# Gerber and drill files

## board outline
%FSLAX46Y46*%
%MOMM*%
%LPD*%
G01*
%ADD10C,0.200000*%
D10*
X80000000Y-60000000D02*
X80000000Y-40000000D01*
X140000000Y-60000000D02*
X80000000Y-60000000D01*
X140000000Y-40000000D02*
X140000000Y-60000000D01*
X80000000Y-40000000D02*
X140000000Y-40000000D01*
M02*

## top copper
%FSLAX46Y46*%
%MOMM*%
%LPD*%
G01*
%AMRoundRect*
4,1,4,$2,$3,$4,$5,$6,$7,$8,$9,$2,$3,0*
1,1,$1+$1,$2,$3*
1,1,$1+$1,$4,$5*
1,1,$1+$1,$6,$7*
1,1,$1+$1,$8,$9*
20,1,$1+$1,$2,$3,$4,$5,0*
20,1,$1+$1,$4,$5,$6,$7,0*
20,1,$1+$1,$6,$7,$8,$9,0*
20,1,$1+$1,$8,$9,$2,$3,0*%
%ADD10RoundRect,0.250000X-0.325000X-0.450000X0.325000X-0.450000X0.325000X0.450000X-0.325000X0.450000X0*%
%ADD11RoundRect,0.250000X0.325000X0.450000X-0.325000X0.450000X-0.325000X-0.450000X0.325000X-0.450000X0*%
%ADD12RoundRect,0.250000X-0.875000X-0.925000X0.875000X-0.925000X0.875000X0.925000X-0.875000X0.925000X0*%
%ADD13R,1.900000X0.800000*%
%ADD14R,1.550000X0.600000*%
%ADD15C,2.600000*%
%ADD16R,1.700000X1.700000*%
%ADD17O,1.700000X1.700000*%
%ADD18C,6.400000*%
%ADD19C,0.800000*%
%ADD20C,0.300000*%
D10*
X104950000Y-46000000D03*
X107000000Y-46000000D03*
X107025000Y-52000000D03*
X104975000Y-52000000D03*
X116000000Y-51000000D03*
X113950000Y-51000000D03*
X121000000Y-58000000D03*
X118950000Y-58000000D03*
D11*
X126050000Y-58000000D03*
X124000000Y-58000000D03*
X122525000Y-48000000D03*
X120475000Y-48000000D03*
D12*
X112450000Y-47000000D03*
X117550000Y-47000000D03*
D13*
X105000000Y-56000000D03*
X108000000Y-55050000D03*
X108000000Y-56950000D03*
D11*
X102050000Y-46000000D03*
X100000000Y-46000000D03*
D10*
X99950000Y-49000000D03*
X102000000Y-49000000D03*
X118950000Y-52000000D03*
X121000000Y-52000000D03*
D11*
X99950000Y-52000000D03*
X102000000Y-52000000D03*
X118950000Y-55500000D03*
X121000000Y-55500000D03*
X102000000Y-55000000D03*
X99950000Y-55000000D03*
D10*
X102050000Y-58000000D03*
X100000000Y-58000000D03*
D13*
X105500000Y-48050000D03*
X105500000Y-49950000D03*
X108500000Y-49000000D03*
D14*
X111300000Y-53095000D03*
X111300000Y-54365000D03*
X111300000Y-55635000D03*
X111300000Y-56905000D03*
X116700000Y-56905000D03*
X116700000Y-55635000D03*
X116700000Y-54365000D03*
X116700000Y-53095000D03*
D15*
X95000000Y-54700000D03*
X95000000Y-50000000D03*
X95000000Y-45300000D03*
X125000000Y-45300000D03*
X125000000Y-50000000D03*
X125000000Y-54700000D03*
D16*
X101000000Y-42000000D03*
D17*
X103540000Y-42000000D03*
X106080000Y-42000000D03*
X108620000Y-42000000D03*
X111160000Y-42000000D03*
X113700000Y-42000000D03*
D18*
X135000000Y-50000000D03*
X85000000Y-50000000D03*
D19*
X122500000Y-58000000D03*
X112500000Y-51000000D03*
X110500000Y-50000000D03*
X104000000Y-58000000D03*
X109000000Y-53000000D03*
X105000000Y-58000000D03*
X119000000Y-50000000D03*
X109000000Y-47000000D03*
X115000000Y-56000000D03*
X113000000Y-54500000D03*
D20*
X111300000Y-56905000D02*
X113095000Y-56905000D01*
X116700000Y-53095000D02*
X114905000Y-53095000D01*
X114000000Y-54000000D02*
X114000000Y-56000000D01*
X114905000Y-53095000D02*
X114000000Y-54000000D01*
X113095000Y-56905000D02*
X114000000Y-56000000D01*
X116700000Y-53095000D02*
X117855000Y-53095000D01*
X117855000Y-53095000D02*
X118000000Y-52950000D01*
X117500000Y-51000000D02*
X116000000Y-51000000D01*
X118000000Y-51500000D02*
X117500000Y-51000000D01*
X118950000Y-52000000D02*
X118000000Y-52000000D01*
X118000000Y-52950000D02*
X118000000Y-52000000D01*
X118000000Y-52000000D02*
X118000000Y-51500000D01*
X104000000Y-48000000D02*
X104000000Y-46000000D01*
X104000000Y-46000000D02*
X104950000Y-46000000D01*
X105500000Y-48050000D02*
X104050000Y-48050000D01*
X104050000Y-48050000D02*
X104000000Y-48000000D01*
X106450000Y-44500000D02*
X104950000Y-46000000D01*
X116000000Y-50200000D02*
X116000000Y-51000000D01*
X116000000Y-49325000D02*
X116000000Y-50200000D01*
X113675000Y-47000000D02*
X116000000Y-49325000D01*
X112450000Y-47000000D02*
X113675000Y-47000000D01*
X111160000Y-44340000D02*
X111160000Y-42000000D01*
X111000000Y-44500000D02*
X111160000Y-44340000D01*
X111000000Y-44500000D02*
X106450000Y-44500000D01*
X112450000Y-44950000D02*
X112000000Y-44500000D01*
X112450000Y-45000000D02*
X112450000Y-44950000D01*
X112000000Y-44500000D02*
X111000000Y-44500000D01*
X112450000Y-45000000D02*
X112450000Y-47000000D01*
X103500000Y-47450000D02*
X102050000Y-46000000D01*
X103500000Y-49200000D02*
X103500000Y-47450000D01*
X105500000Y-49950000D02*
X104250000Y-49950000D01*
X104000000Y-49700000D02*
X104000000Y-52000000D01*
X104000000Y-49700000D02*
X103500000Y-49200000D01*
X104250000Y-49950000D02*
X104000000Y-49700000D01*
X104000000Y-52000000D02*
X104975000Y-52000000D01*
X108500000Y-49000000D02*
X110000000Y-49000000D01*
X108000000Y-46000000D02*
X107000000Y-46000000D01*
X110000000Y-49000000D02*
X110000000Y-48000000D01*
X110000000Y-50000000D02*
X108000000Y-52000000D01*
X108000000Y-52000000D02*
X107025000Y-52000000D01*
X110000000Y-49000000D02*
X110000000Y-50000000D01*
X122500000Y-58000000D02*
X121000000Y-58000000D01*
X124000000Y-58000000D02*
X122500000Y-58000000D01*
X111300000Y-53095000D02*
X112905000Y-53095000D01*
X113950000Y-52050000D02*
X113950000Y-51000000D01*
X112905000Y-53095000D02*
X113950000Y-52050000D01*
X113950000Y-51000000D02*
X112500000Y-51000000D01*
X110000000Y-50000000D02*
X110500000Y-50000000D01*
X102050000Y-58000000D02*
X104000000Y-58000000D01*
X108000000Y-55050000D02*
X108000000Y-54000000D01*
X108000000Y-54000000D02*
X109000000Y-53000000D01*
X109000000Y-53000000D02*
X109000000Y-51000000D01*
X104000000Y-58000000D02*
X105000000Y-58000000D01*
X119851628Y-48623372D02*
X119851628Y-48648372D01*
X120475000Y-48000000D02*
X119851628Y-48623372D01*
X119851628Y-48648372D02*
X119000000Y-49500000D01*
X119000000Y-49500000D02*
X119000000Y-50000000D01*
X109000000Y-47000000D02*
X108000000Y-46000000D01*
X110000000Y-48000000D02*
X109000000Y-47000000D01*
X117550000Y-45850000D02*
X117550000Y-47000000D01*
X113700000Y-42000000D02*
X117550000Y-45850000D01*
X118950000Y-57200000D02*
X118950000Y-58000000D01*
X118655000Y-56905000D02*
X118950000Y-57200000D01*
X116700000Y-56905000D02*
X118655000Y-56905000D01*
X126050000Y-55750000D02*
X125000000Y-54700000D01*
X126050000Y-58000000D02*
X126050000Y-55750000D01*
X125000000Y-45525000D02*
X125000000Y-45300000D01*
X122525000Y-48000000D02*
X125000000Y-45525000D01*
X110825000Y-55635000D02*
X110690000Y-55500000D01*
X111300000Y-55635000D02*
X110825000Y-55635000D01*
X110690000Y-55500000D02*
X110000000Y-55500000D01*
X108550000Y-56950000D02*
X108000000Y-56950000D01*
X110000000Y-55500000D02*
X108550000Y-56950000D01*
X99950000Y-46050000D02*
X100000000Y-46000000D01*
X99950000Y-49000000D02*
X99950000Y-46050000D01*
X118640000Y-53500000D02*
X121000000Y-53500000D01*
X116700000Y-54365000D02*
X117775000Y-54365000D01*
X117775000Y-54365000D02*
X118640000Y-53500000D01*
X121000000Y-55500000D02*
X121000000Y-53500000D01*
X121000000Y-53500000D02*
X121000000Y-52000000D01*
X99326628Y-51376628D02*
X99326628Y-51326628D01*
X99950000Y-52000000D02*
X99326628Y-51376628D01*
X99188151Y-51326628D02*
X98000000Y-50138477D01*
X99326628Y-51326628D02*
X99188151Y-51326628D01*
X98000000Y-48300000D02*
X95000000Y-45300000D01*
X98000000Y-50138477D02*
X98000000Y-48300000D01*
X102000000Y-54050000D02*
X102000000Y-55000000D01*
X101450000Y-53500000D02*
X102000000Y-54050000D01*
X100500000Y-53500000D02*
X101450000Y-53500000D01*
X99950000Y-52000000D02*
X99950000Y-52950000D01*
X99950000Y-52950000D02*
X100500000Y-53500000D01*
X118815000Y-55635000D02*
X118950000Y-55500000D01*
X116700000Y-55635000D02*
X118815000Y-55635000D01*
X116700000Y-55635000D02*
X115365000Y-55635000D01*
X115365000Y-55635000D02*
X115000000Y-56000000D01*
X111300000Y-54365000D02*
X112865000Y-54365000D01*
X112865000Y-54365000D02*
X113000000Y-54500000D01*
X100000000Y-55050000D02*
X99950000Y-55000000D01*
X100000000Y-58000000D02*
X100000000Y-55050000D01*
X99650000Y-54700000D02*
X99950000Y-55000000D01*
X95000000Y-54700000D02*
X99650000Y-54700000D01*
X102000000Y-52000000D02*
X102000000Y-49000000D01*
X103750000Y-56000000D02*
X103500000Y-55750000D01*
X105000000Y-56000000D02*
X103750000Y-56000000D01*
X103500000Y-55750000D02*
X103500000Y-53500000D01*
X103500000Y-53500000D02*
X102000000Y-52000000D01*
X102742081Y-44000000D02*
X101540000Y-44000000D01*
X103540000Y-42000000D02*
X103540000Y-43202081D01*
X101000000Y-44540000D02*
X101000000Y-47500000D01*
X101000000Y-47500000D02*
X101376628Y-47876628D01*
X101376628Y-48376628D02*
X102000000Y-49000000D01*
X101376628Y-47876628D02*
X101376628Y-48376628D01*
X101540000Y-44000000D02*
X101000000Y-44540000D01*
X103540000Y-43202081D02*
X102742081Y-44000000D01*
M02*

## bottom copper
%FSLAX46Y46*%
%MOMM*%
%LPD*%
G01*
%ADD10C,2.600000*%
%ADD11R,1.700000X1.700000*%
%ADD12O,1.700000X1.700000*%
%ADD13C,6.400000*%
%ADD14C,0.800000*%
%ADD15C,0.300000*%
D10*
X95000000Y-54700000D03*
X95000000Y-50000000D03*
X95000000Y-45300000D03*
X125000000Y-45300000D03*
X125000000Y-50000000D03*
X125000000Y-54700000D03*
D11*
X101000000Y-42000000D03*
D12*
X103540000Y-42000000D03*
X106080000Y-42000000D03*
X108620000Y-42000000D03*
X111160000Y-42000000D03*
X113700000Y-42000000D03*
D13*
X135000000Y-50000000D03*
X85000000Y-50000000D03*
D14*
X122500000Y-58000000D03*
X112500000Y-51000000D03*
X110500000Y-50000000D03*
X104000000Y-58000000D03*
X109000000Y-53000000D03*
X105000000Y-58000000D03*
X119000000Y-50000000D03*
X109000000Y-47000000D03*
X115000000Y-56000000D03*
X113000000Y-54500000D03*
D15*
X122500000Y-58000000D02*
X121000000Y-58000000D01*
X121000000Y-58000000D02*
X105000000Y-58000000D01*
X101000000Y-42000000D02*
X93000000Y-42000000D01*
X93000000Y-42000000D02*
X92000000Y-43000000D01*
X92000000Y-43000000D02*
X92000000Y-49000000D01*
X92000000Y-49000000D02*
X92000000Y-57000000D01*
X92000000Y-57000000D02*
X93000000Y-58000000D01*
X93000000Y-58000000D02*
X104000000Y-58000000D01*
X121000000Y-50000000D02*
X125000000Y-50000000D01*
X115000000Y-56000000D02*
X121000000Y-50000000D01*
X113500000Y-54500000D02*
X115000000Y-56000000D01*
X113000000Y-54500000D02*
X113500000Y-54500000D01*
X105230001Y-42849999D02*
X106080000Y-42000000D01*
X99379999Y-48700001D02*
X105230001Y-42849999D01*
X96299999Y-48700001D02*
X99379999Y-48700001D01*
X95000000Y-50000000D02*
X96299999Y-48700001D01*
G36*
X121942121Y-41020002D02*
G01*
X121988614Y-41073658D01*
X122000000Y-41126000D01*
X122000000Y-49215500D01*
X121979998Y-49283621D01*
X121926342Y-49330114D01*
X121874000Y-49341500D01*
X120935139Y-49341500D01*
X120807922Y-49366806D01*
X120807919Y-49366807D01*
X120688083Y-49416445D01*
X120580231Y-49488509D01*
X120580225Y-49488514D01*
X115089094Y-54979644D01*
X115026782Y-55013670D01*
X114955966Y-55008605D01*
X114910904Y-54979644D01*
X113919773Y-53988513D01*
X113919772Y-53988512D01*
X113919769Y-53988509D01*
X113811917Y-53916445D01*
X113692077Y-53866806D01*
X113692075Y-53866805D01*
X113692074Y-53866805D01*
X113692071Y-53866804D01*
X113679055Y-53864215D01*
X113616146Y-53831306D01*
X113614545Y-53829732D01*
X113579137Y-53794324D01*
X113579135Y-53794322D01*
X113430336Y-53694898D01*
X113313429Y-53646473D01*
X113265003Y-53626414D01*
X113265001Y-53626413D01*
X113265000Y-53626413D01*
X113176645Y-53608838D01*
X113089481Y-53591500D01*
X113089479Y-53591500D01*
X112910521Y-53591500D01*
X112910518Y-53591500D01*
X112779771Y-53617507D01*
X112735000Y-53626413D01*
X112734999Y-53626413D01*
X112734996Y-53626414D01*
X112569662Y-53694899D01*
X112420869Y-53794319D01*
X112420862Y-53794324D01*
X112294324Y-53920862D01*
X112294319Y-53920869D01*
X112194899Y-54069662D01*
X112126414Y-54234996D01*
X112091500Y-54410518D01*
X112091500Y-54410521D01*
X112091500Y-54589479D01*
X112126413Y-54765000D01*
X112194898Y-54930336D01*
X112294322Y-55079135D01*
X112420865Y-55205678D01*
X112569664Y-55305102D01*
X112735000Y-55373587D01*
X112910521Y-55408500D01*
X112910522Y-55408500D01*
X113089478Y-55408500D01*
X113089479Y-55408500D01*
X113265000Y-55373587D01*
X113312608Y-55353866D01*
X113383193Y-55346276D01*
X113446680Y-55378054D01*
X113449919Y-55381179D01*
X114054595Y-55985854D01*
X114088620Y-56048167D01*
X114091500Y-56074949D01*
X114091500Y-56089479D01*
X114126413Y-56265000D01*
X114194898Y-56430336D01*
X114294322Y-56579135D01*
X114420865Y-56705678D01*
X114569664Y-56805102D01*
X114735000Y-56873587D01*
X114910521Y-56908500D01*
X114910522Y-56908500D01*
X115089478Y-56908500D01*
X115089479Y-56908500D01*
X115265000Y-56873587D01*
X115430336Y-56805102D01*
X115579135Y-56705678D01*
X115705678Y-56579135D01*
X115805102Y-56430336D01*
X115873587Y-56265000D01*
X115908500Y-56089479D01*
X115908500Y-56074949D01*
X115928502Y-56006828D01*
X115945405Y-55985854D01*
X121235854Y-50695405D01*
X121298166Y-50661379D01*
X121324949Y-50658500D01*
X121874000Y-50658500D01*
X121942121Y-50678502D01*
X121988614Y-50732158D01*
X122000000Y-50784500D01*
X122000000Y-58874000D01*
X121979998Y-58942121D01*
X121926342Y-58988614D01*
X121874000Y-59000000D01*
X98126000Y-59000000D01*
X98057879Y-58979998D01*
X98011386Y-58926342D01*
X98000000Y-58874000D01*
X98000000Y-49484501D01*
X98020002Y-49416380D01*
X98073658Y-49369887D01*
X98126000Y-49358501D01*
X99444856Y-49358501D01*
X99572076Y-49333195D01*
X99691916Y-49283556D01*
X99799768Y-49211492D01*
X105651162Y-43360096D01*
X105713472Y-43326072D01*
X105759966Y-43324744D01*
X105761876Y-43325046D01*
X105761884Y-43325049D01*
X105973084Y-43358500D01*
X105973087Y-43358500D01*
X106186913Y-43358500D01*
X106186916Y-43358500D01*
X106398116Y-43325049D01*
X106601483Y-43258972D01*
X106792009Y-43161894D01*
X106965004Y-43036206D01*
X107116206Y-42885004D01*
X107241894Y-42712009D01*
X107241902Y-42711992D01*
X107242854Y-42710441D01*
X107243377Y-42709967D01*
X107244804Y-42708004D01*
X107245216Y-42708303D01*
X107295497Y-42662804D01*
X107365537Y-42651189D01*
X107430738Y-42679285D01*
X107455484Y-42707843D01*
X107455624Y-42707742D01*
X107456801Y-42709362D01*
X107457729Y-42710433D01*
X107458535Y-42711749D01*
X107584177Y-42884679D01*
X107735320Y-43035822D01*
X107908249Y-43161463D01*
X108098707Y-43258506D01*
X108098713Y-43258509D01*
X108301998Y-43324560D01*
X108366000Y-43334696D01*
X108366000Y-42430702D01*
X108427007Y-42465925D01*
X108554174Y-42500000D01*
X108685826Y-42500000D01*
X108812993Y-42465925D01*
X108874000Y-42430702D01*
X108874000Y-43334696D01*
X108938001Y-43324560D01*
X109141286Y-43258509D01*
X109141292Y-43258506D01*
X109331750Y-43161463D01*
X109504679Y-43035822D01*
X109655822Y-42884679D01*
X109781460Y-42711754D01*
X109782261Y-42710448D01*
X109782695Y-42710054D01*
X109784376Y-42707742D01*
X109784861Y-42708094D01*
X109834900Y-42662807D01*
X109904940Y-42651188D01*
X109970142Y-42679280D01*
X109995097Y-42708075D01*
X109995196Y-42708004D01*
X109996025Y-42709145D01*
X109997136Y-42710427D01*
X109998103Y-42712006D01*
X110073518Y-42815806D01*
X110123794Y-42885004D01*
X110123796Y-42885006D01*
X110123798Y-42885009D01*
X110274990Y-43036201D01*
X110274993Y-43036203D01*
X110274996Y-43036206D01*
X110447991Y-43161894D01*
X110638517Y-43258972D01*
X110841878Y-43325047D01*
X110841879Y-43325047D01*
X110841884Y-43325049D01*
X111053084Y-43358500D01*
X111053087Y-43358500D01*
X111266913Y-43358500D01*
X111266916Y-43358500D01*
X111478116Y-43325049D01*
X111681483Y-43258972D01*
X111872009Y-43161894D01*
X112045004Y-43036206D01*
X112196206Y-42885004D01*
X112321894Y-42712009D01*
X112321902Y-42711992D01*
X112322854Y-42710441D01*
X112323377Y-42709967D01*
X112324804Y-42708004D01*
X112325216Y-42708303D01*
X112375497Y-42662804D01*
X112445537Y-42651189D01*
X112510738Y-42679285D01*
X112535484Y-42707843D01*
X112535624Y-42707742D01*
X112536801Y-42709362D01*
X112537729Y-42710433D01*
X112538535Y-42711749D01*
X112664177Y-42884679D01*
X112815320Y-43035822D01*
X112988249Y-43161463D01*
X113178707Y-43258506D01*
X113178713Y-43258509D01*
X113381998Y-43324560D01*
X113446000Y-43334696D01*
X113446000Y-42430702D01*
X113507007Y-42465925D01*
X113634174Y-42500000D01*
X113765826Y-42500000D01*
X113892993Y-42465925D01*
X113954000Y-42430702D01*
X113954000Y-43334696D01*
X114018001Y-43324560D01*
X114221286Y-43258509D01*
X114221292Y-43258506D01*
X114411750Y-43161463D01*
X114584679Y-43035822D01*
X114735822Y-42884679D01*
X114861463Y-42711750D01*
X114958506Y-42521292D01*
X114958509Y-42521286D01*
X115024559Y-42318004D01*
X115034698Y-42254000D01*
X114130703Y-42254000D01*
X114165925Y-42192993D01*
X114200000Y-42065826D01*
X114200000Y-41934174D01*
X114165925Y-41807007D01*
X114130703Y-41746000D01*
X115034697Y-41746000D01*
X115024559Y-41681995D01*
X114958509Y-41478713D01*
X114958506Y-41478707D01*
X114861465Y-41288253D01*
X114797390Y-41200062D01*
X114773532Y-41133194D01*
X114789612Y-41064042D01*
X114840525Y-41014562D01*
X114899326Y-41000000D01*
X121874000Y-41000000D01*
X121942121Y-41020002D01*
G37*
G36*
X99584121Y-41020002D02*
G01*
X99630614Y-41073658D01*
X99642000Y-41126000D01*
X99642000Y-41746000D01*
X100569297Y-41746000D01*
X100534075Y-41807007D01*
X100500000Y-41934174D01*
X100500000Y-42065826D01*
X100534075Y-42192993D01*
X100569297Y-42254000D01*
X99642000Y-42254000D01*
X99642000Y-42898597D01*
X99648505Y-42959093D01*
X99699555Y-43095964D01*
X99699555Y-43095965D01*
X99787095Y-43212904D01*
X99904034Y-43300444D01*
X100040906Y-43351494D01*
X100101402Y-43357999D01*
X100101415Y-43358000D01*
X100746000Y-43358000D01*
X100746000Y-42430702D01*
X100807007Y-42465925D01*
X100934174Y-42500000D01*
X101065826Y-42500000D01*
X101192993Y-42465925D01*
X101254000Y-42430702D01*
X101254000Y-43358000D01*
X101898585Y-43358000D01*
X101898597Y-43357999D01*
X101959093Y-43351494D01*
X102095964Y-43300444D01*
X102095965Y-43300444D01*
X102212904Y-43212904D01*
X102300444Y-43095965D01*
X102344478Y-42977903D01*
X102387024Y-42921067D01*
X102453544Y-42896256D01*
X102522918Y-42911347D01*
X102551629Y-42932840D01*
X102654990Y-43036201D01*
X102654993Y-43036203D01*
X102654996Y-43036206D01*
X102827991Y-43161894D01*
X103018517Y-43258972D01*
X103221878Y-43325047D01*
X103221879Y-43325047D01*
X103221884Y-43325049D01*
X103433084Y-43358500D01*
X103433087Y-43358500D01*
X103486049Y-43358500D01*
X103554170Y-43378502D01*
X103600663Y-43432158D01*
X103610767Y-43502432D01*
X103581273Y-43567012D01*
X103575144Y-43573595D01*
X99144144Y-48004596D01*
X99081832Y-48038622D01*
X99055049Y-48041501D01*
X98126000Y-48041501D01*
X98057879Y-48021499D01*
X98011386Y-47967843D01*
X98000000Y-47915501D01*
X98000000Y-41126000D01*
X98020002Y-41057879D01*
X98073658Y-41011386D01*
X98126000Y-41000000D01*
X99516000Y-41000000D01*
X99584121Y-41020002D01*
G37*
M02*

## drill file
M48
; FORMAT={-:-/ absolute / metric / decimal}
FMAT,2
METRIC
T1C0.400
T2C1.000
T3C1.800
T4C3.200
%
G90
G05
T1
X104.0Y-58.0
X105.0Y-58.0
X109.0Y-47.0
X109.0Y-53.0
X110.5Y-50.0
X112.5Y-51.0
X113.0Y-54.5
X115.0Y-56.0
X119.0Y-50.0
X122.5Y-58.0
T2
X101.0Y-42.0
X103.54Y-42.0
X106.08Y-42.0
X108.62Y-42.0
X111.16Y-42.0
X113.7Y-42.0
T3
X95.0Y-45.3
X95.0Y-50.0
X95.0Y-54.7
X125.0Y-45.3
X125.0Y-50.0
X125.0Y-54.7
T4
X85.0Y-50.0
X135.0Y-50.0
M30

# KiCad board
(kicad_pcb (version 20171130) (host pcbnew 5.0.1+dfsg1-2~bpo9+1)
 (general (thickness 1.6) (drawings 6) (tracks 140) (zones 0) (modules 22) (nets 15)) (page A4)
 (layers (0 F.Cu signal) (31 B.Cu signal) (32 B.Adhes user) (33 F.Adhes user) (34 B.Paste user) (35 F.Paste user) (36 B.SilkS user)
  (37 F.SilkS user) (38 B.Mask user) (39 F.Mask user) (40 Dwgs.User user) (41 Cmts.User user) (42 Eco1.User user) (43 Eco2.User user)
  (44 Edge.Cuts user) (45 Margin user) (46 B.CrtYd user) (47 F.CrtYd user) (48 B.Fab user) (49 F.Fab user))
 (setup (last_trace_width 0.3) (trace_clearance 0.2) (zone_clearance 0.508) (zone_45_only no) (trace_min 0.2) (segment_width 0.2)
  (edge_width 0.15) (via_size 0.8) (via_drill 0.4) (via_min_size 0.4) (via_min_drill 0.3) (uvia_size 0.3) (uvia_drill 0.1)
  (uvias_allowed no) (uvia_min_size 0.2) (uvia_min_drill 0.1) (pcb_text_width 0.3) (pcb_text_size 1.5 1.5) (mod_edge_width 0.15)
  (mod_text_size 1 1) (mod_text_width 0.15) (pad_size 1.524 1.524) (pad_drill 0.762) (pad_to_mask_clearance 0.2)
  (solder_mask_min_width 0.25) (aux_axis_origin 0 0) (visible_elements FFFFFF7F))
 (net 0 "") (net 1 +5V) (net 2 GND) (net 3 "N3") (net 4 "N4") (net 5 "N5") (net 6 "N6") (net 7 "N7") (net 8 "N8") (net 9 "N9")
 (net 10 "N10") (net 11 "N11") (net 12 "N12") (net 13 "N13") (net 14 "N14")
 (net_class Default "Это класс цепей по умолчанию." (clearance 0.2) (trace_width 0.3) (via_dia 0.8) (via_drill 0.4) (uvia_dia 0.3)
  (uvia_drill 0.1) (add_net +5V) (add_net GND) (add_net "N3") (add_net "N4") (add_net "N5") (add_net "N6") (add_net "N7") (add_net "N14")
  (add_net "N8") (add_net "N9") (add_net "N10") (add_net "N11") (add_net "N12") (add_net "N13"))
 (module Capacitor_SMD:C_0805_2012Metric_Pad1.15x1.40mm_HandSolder (layer F.Cu) (at 105.975 46)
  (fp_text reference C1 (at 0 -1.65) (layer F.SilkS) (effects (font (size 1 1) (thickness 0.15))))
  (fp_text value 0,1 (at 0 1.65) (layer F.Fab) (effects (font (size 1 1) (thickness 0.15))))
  (pad 1 smd roundrect (at -1.025 0) (size 1.15 1.4) (layers F.Cu F.Paste F.Mask) (roundrect_rratio 0.217391) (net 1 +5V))
  (pad 2 smd roundrect (at 1.025 0) (size 1.15 1.4) (layers F.Cu F.Paste F.Mask) (roundrect_rratio 0.217391) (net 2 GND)))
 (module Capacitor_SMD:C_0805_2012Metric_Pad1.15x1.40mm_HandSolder (layer F.Cu) (at 106 52)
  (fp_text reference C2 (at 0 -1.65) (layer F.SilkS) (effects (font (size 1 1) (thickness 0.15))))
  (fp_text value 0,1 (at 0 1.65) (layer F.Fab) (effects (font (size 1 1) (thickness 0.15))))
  (pad 2 smd roundrect (at 1.025 0) (size 1.15 1.4) (layers F.Cu F.Paste F.Mask) (roundrect_rratio 0.217391) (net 2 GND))
  (pad 1 smd roundrect (at -1.025 0) (size 1.15 1.4) (layers F.Cu F.Paste F.Mask) (roundrect_rratio 0.217391) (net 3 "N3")))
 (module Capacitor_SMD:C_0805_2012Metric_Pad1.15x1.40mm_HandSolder (layer F.Cu) (at 114.975 51)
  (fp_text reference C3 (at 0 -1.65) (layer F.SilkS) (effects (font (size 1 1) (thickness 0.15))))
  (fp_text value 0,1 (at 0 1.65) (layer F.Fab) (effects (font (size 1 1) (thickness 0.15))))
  (pad 2 smd roundrect (at 1.025 0) (size 1.15 1.4) (layers F.Cu F.Paste F.Mask) (roundrect_rratio 0.217391) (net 1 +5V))
  (pad 1 smd roundrect (at -1.025 0) (size 1.15 1.4) (layers F.Cu F.Paste F.Mask) (roundrect_rratio 0.217391) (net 2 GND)))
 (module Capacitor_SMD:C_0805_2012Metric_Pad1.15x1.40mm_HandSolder (layer F.Cu) (at 119.975 58)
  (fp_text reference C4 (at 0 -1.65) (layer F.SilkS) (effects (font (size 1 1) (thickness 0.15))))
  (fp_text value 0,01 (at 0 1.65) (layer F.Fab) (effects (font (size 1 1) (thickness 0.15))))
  (pad 2 smd roundrect (at 1.025 0) (size 1.15 1.4) (layers F.Cu F.Paste F.Mask) (roundrect_rratio 0.217391) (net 2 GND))
  (pad 1 smd roundrect (at -1.025 0) (size 1.15 1.4) (layers F.Cu F.Paste F.Mask) (roundrect_rratio 0.217391) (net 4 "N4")))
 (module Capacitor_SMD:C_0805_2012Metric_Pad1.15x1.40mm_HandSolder (layer F.Cu) (at 125.025 58 180)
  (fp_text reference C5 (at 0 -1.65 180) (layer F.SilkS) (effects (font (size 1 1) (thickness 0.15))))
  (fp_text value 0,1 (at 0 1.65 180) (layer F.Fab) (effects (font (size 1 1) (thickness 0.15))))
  (pad 1 smd roundrect (at -1.025 0 180) (size 1.15 1.4) (layers F.Cu F.Paste F.Mask) (roundrect_rratio 0.217391) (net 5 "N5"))
  (pad 2 smd roundrect (at 1.025 0 180) (size 1.15 1.4) (layers F.Cu F.Paste F.Mask) (roundrect_rratio 0.217391) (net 2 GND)))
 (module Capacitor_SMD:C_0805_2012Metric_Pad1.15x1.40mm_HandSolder (layer F.Cu) (at 121.5 48 180)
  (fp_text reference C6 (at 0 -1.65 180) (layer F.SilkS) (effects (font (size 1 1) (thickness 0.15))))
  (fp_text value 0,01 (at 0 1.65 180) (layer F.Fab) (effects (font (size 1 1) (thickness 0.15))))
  (pad 1 smd roundrect (at -1.025 0 180) (size 1.15 1.4) (layers F.Cu F.Paste F.Mask) (roundrect_rratio 0.217391) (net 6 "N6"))
  (pad 2 smd roundrect (at 1.025 0 180) (size 1.15 1.4) (layers F.Cu F.Paste F.Mask) (roundrect_rratio 0.217391) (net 2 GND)))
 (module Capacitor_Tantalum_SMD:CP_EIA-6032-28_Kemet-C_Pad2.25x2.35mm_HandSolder (layer F.Cu) (at 115 47)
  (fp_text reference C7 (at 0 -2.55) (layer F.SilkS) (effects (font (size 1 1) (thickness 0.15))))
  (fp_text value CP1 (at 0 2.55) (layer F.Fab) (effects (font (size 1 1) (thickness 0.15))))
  (pad 1 smd roundrect (at -2.55 0) (size 2.25 2.35) (layers F.Cu F.Paste F.Mask) (roundrect_rratio 0.111111) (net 1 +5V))
  (pad 2 smd roundrect (at 2.55 0) (size 2.25 2.35) (layers F.Cu F.Paste F.Mask) (roundrect_rratio 0.111111) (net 2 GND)))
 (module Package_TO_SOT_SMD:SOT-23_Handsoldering (layer F.Cu) (at 106.5 56 180)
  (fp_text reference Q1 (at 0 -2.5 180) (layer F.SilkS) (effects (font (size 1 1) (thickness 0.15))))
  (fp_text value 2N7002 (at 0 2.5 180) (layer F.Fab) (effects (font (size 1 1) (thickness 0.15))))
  (pad 3 smd rect (at 1.5 0 180) (size 1.9 0.8) (layers F.Cu F.Paste F.Mask) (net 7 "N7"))
  (pad 2 smd rect (at -1.5 0.95 180) (size 1.9 0.8) (layers F.Cu F.Paste F.Mask) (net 2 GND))
  (pad 1 smd rect (at -1.5 -0.95 180) (size 1.9 0.8) (layers F.Cu F.Paste F.Mask) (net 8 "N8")))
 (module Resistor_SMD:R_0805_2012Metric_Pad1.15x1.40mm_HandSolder (layer F.Cu) (at 101.025 46 180)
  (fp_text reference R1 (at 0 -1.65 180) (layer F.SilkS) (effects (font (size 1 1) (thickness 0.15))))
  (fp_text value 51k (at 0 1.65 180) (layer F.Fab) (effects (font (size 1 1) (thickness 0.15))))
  (pad 1 smd roundrect (at -1.025 0 180) (size 1.15 1.4) (layers F.Cu F.Paste F.Mask) (roundrect_rratio 0.217391) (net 3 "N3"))
  (pad 2 smd roundrect (at 1.025 0 180) (size 1.15 1.4) (layers F.Cu F.Paste F.Mask) (roundrect_rratio 0.217391) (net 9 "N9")))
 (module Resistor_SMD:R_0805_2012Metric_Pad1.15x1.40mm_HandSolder (layer F.Cu) (at 100.975 49)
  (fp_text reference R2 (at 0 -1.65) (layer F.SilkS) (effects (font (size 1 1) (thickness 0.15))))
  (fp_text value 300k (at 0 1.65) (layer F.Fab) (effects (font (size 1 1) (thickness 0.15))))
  (pad 1 smd roundrect (at -1.025 0) (size 1.15 1.4) (layers F.Cu F.Paste F.Mask) (roundrect_rratio 0.217391) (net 9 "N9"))
  (pad 2 smd roundrect (at 1.025 0) (size 1.15 1.4) (layers F.Cu F.Paste F.Mask) (roundrect_rratio 0.217391) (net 7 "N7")))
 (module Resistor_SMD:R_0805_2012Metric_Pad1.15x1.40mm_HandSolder (layer F.Cu) (at 119.975 52)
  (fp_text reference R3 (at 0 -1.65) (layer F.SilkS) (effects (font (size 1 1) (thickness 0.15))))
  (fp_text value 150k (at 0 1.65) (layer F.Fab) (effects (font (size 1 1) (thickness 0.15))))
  (pad 1 smd roundrect (at -1.025 0) (size 1.15 1.4) (layers F.Cu F.Paste F.Mask) (roundrect_rratio 0.217391) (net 1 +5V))
  (pad 2 smd roundrect (at 1.025 0) (size 1.15 1.4) (layers F.Cu F.Paste F.Mask) (roundrect_rratio 0.217391) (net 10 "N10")))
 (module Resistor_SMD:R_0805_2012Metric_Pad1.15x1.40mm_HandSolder (layer F.Cu) (at 100.975 52 180)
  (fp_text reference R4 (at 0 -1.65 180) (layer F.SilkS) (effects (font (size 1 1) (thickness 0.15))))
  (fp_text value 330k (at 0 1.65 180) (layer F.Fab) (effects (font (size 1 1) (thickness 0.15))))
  (pad 2 smd roundrect (at 1.025 0 180) (size 1.15 1.4) (layers F.Cu F.Paste F.Mask) (roundrect_rratio 0.217391) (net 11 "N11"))
  (pad 1 smd roundrect (at -1.025 0 180) (size 1.15 1.4) (layers F.Cu F.Paste F.Mask) (roundrect_rratio 0.217391) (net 7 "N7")))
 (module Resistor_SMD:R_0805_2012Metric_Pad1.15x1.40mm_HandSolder (layer F.Cu) (at 119.975 55.5 180)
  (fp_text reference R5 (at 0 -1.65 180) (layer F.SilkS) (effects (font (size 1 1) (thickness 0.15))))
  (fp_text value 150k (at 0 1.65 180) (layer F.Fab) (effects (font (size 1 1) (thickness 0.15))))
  (pad 2 smd roundrect (at 1.025 0 180) (size 1.15 1.4) (layers F.Cu F.Paste F.Mask) (roundrect_rratio 0.217391) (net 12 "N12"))
  (pad 1 smd roundrect (at -1.025 0 180) (size 1.15 1.4) (layers F.Cu F.Paste F.Mask) (roundrect_rratio 0.217391) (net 10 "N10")))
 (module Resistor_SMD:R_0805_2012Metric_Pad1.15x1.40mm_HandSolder (layer F.Cu) (at 100.975 55 180)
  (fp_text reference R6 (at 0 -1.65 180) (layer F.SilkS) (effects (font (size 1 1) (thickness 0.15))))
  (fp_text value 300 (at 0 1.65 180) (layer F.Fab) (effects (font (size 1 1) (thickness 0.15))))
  (pad 1 smd roundrect (at -1.025 0 180) (size 1.15 1.4) (layers F.Cu F.Paste F.Mask) (roundrect_rratio 0.217391) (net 11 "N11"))
  (pad 2 smd roundrect (at 1.025 0 180) (size 1.15 1.4) (layers F.Cu F.Paste F.Mask) (roundrect_rratio 0.217391) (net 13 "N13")))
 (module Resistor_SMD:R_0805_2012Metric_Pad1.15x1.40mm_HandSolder (layer F.Cu) (at 101.025 58)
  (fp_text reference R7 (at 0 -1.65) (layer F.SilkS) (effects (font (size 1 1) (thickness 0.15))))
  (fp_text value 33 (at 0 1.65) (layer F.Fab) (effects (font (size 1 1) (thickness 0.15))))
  (pad 2 smd roundrect (at 1.025 0) (size 1.15 1.4) (layers F.Cu F.Paste F.Mask) (roundrect_rratio 0.217391) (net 2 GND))
  (pad 1 smd roundrect (at -1.025 0) (size 1.15 1.4) (layers F.Cu F.Paste F.Mask) (roundrect_rratio 0.217391) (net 13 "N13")))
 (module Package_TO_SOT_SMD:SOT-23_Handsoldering (layer F.Cu) (at 107 49)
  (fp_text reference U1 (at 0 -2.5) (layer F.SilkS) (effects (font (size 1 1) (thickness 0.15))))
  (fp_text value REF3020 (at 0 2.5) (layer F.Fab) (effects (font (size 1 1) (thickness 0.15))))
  (pad 1 smd rect (at -1.5 -0.95) (size 1.9 0.8) (layers F.Cu F.Paste F.Mask) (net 1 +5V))
  (pad 2 smd rect (at -1.5 0.95) (size 1.9 0.8) (layers F.Cu F.Paste F.Mask) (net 3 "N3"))
  (pad 3 smd rect (at 1.5 0) (size 1.9 0.8) (layers F.Cu F.Paste F.Mask) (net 2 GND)))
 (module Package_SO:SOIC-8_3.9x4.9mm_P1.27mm (layer F.Cu) (at 114 55)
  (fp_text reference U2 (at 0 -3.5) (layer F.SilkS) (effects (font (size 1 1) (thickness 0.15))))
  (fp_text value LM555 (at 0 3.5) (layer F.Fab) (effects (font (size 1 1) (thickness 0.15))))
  (pad 1 smd rect (at -2.7 -1.905) (size 1.55 0.6) (layers F.Cu F.Paste F.Mask) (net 2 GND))
  (pad 2 smd rect (at -2.7 -0.635) (size 1.55 0.6) (layers F.Cu F.Paste F.Mask) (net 12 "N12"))
  (pad 3 smd rect (at -2.7 0.635) (size 1.55 0.6) (layers F.Cu F.Paste F.Mask) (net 8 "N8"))
  (pad 4 smd rect (at -2.7 1.905) (size 1.55 0.6) (layers F.Cu F.Paste F.Mask) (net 1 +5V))
  (pad 5 smd rect (at 2.7 1.905) (size 1.55 0.6) (layers F.Cu F.Paste F.Mask) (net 4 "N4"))
  (pad 6 smd rect (at 2.7 0.635) (size 1.55 0.6) (layers F.Cu F.Paste F.Mask) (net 12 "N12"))
  (pad 7 smd rect (at 2.7 -0.635) (size 1.55 0.6) (layers F.Cu F.Paste F.Mask) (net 10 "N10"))
  (pad 8 smd rect (at 2.7 -1.905) (size 1.55 0.6) (layers F.Cu F.Paste F.Mask) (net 1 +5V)))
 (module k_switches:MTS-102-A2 (layer B.Cu) (at 95 50 270)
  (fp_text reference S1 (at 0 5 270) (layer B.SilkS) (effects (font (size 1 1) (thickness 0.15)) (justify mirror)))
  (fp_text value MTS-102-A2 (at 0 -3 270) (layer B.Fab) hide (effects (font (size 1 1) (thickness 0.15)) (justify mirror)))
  (pad 3 thru_hole circle (at 4.7 0 270) (size 2.6 2.6) (drill 1.8) (layers *.Cu *.Mask) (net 13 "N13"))
  (pad 2 thru_hole circle (at 0 0 270) (size 2.6 2.6) (drill 1.8) (layers *.Cu *.Mask) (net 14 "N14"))
  (pad 1 thru_hole circle (at -4.7 0 270) (size 2.6 2.6) (drill 1.8) (layers *.Cu *.Mask) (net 11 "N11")))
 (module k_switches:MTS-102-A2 (layer B.Cu) (at 125 50 270)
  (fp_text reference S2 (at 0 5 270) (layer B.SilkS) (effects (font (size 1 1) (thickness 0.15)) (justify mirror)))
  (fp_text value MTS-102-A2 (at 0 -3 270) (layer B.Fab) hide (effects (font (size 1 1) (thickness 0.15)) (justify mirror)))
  (pad 1 thru_hole circle (at -4.7 0 270) (size 2.6 2.6) (drill 1.8) (layers *.Cu *.Mask) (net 6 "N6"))
  (pad 2 thru_hole circle (at 0 0 270) (size 2.6 2.6) (drill 1.8) (layers *.Cu *.Mask) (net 12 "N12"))
  (pad 3 thru_hole circle (at 4.7 0 270) (size 2.6 2.6) (drill 1.8) (layers *.Cu *.Mask) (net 5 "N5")))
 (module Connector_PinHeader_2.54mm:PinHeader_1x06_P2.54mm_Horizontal (layer F.Cu) (at 101 42 90)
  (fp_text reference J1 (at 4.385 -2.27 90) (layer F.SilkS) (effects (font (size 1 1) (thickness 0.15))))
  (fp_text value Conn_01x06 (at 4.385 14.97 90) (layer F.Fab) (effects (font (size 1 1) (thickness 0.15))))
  (pad 1 thru_hole rect (at 0 0 90) (size 1.7 1.7) (drill 1) (layers *.Cu *.Mask) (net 2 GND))
  (pad 2 thru_hole oval (at 0 2.54 90) (size 1.7 1.7) (drill 1) (layers *.Cu *.Mask) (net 7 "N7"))
  (pad 3 thru_hole oval (at 0 5.08 90) (size 1.7 1.7) (drill 1) (layers *.Cu *.Mask) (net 14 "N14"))
  (pad 4 thru_hole oval (at 0 7.62 90) (size 1.7 1.7) (drill 1) (layers *.Cu *.Mask) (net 2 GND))
  (pad 5 thru_hole oval (at 0 10.16 90) (size 1.7 1.7) (drill 1) (layers *.Cu *.Mask) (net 1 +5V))
  (pad 6 thru_hole oval (at 0 12.7 90) (size 1.7 1.7) (drill 1) (layers *.Cu *.Mask) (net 2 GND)))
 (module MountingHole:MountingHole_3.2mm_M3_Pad (layer F.Cu) (at 135 50)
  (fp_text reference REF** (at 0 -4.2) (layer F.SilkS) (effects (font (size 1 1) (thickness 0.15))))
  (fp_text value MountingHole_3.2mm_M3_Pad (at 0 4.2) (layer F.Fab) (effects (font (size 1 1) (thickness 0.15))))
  (pad 1 thru_hole circle (at 0 0) (size 6.4 6.4) (drill 3.2) (layers *.Cu *.Mask)))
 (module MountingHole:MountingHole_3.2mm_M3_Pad (layer F.Cu) (at 85 50)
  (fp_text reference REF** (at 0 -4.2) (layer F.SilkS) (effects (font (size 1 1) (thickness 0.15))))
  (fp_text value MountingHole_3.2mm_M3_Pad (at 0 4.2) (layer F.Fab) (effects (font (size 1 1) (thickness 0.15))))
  (pad 1 thru_hole circle (at 0 0) (size 6.4 6.4) (drill 3.2) (layers *.Cu *.Mask)))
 (gr_line (start 80 60) (end 80 40) (layer Edge.Cuts) (width 0.2))
 (gr_line (start 140 60) (end 80 60) (layer Edge.Cuts) (width 0.2))
 (gr_line (start 140 40) (end 140 60) (layer Edge.Cuts) (width 0.2))
 (gr_line (start 80 40) (end 140 40) (layer Edge.Cuts) (width 0.2))
 (segment (start 111.3 56.905) (end 113.095 56.905) (width 0.3) (layer F.Cu) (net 1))
 (segment (start 116.7 53.095) (end 114.905 53.095) (width 0.3) (layer F.Cu) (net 1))
 (segment (start 114 54) (end 114 56) (width 0.3) (layer F.Cu) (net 1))
 (segment (start 114.905 53.095) (end 114 54) (width 0.3) (layer F.Cu) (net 1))
 (segment (start 113.095 56.905) (end 114 56) (width 0.3) (layer F.Cu) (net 1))
 (segment (start 116.7 53.095) (end 117.855 53.095) (width 0.3) (layer F.Cu) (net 1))
 (segment (start 117.855 53.095) (end 118 52.95) (width 0.3) (layer F.Cu) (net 1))
 (segment (start 117.5 51) (end 116 51) (width 0.3) (layer F.Cu) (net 1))
 (segment (start 118 51.5) (end 117.5 51) (width 0.3) (layer F.Cu) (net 1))
 (segment (start 118.95 52) (end 118 52) (width 0.3) (layer F.Cu) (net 1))
 (segment (start 118 52.95) (end 118 52) (width 0.3) (layer F.Cu) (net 1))
 (segment (start 118 52) (end 118 51.5) (width 0.3) (layer F.Cu) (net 1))
 (segment (start 104 48) (end 104 46) (width 0.3) (layer F.Cu) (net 1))
 (segment (start 104 46) (end 104.95 46) (width 0.3) (layer F.Cu) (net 1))
 (segment (start 105.5 48.05) (end 104.05 48.05) (width 0.3) (layer F.Cu) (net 1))
 (segment (start 104.05 48.05) (end 104 48) (width 0.3) (layer F.Cu) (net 1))
 (segment (start 106.45 44.5) (end 104.95 46) (width 0.3) (layer F.Cu) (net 1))
 (segment (start 116 50.2) (end 116 51) (width 0.3) (layer F.Cu) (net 1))
 (segment (start 116 49.325) (end 116 50.2) (width 0.3) (layer F.Cu) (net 1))
 (segment (start 113.675 47) (end 116 49.325) (width 0.3) (layer F.Cu) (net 1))
 (segment (start 112.45 47) (end 113.675 47) (width 0.3) (layer F.Cu) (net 1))
 (segment (start 111.16 44.34) (end 111.16 42) (width 0.3) (layer F.Cu) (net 1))
 (segment (start 111 44.5) (end 111.16 44.34) (width 0.3) (layer F.Cu) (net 1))
 (segment (start 111 44.5) (end 106.45 44.5) (width 0.3) (layer F.Cu) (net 1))
 (segment (start 112.45 44.95) (end 112 44.5) (width 0.3) (layer F.Cu) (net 1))
 (segment (start 112.45 45) (end 112.45 44.95) (width 0.3) (layer F.Cu) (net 1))
 (segment (start 112 44.5) (end 111 44.5) (width 0.3) (layer F.Cu) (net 1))
 (segment (start 112.45 45) (end 112.45 47) (width 0.3) (layer F.Cu) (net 1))
 (segment (start 103.5 47.45) (end 102.05 46) (width 0.3) (layer F.Cu) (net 3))
 (segment (start 103.5 49.2) (end 103.5 47.45) (width 0.3) (layer F.Cu) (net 3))
 (segment (start 105.5 49.95) (end 104.25 49.95) (width 0.3) (layer F.Cu) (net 3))
 (segment (start 104 49.7) (end 104 52) (width 0.3) (layer F.Cu) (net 3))
 (segment (start 104 49.7) (end 103.5 49.2) (width 0.3) (layer F.Cu) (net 3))
 (segment (start 104.25 49.95) (end 104 49.7) (width 0.3) (layer F.Cu) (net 3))
 (segment (start 104 52) (end 104.975 52) (width 0.3) (layer F.Cu) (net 3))
 (segment (start 108.5 49) (end 110 49) (width 0.3) (layer F.Cu) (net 2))
 (segment (start 108 46) (end 107 46) (width 0.3) (layer F.Cu) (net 2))
 (segment (start 110 49) (end 110 48) (width 0.3) (layer F.Cu) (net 2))
 (segment (start 110 50) (end 108 52) (width 0.3) (layer F.Cu) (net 2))
 (segment (start 108 52) (end 107.025 52) (width 0.3) (layer F.Cu) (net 2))
 (segment (start 110 49) (end 110 50) (width 0.3) (layer F.Cu) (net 2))
 (via (at 122.5 58) (size 0.8) (drill 0.4) (layers F.Cu B.Cu) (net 2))
 (segment (start 122.5 58) (end 121 58) (width 0.3) (layer F.Cu) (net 2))
 (segment (start 124 58) (end 122.5 58) (width 0.3) (layer F.Cu) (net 2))
 (segment (start 111.3 53.095) (end 112.905 53.095) (width 0.3) (layer F.Cu) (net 2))
 (segment (start 113.95 52.05) (end 113.95 51) (width 0.3) (layer F.Cu) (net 2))
 (segment (start 112.905 53.095) (end 113.95 52.05) (width 0.3) (layer F.Cu) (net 2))
 (via (at 112.5 51) (size 0.8) (drill 0.4) (layers F.Cu B.Cu) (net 2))
 (segment (start 113.95 51) (end 112.5 51) (width 0.3) (layer F.Cu) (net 2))
 (via (at 110.5 50) (size 0.8) (drill 0.4) (layers F.Cu B.Cu) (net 2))
 (segment (start 110 50) (end 110.5 50) (width 0.3) (layer F.Cu) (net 2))
 (via (at 104 58) (size 0.8) (drill 0.4) (layers F.Cu B.Cu) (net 2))
 (segment (start 102.05 58) (end 104 58) (width 0.3) (layer F.Cu) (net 2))
 (via (at 109 53) (size 0.8) (drill 0.4) (layers F.Cu B.Cu) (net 2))
 (segment (start 108 55.05) (end 108 54) (width 0.3) (layer F.Cu) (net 2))
 (segment (start 108 54) (end 109 53) (width 0.3) (layer F.Cu) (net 2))
 (segment (start 109 53) (end 109 51) (width 0.3) (layer F.Cu) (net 2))
 (via (at 105 58) (size 0.8) (drill 0.4) (layers F.Cu B.Cu) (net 2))
 (segment (start 104 58) (end 105 58) (width 0.3) (layer F.Cu) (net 2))
 (segment (start 119.851628 48.623372) (end 119.851628 48.648372) (width 0.3) (layer F.Cu) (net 2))
 (segment (start 120.475 48) (end 119.851628 48.623372) (width 0.3) (layer F.Cu) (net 2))
 (via (at 119 50) (size 0.8) (drill 0.4) (layers F.Cu B.Cu) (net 2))
 (segment (start 119.851628 48.648372) (end 119 49.5) (width 0.3) (layer F.Cu) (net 2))
 (segment (start 119 49.5) (end 119 50) (width 0.3) (layer F.Cu) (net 2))
 (segment (start 122.5 58) (end 121 58) (width 0.3) (layer B.Cu) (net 2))
 (segment (start 121 58) (end 105 58) (width 0.3) (layer B.Cu) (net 2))
 (via (at 109 47) (size 0.8) (drill 0.4) (layers F.Cu B.Cu) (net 2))
 (segment (start 109 47) (end 108 46) (width 0.3) (layer F.Cu) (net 2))
 (segment (start 110 48) (end 109 47) (width 0.3) (layer F.Cu) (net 2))
 (segment (start 117.55 45.85) (end 117.55 47) (width 0.3) (layer F.Cu) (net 2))
 (segment (start 113.7 42) (end 117.55 45.85) (width 0.3) (layer F.Cu) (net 2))
 (segment (start 101 42) (end 93 42) (width 0.3) (layer B.Cu) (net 2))
 (segment (start 93 42) (end 92 43) (width 0.3) (layer B.Cu) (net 2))
 (segment (start 92 43) (end 92 49) (width 0.3) (layer B.Cu) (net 2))
 (segment (start 92 49) (end 92 57) (width 0.3) (layer B.Cu) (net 2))
 (segment (start 92 57) (end 93 58) (width 0.3) (layer B.Cu) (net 2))
 (segment (start 93 58) (end 104 58) (width 0.3) (layer B.Cu) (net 2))
 (segment (start 118.95 57.2) (end 118.95 58) (width 0.3) (layer F.Cu) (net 4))
 (segment (start 118.655 56.905) (end 118.95 57.2) (width 0.3) (layer F.Cu) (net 4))
 (segment (start 116.7 56.905) (end 118.655 56.905) (width 0.3) (layer F.Cu) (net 4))
 (segment (start 126.05 55.75) (end 125 54.7) (width 0.3) (layer F.Cu) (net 5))
 (segment (start 126.05 58) (end 126.05 55.75) (width 0.3) (layer F.Cu) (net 5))
 (segment (start 125 45.525) (end 125 45.3) (width 0.3) (layer F.Cu) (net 6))
 (segment (start 122.525 48) (end 125 45.525) (width 0.3) (layer F.Cu) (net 6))
 (segment (start 110.825 55.635) (end 110.69 55.5) (width 0.3) (layer F.Cu) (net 8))
 (segment (start 111.3 55.635) (end 110.825 55.635) (width 0.3) (layer F.Cu) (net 8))
 (segment (start 110.69 55.5) (end 110 55.5) (width 0.3) (layer F.Cu) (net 8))
 (segment (start 108.55 56.95) (end 108 56.95) (width 0.3) (layer F.Cu) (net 8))
 (segment (start 110 55.5) (end 108.55 56.95) (width 0.3) (layer F.Cu) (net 8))
 (segment (start 99.95 46.05) (end 100 46) (width 0.3) (layer F.Cu) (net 9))
 (segment (start 99.95 49) (end 99.95 46.05) (width 0.3) (layer F.Cu) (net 9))
 (segment (start 118.64 53.5) (end 121 53.5) (width 0.3) (layer F.Cu) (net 10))
 (segment (start 116.7 54.365) (end 117.775 54.365) (width 0.3) (layer F.Cu) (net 10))
 (segment (start 117.775 54.365) (end 118.64 53.5) (width 0.3) (layer F.Cu) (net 10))
 (segment (start 121 55.5) (end 121 53.5) (width 0.3) (layer F.Cu) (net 10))
 (segment (start 121 53.5) (end 121 52) (width 0.3) (layer F.Cu) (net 10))
 (segment (start 99.326628 51.376628) (end 99.326628 51.326628) (width 0.3) (layer F.Cu) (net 11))
 (segment (start 99.95 52) (end 99.326628 51.376628) (width 0.3) (layer F.Cu) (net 11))
 (segment (start 99.188151 51.326628) (end 98 50.138477) (width 0.3) (layer F.Cu) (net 11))
 (segment (start 99.326628 51.326628) (end 99.188151 51.326628) (width 0.3) (layer F.Cu) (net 11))
 (segment (start 98 48.3) (end 95 45.3) (width 0.3) (layer F.Cu) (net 11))
 (segment (start 98 50.138477) (end 98 48.3) (width 0.3) (layer F.Cu) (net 11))
 (segment (start 102 54.05) (end 102 55) (width 0.3) (layer F.Cu) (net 11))
 (segment (start 101.45 53.5) (end 102 54.05) (width 0.3) (layer F.Cu) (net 11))
 (segment (start 100.5 53.5) (end 101.45 53.5) (width 0.3) (layer F.Cu) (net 11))
 (segment (start 99.95 52) (end 99.95 52.95) (width 0.3) (layer F.Cu) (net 11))
 (segment (start 99.95 52.95) (end 100.5 53.5) (width 0.3) (layer F.Cu) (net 11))
 (segment (start 118.815 55.635) (end 118.95 55.5) (width 0.3) (layer F.Cu) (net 12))
 (segment (start 116.7 55.635) (end 118.815 55.635) (width 0.3) (layer F.Cu) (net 12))
 (via (at 115 56) (size 0.8) (drill 0.4) (layers F.Cu B.Cu) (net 12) (status 1000000))
 (segment (start 116.7 55.635) (end 115.365 55.635) (width 0.3) (layer F.Cu) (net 12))
 (segment (start 115.365 55.635) (end 115 56) (width 0.3) (layer F.Cu) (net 12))
 (segment (start 121 50) (end 125 50) (width 0.3) (layer B.Cu) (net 12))
 (segment (start 115 56) (end 121 50) (width 0.3) (layer B.Cu) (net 12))
 (via (at 113 54.5) (size 0.8) (drill 0.4) (layers F.Cu B.Cu) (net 12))
 (segment (start 111.3 54.365) (end 112.865 54.365) (width 0.3) (layer F.Cu) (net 12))
 (segment (start 112.865 54.365) (end 113 54.5) (width 0.3) (layer F.Cu) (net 12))
 (segment (start 113.5 54.5) (end 115 56) (width 0.3) (layer B.Cu) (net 12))
 (segment (start 113 54.5) (end 113.5 54.5) (width 0.3) (layer B.Cu) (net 12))
 (segment (start 100 55.05) (end 99.95 55) (width 0.3) (layer F.Cu) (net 13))
 (segment (start 100 58) (end 100 55.05) (width 0.3) (layer F.Cu) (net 13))
 (segment (start 99.65 54.7) (end 99.95 55) (width 0.3) (layer F.Cu) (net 13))
 (segment (start 95 54.7) (end 99.65 54.7) (width 0.3) (layer F.Cu) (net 13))
 (segment (start 102 52) (end 102 49) (width 0.3) (layer F.Cu) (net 7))
 (segment (start 103.75 56) (end 103.5 55.75) (width 0.3) (layer F.Cu) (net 7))
 (segment (start 105 56) (end 103.75 56) (width 0.3) (layer F.Cu) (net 7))
 (segment (start 103.5 55.75) (end 103.5 53.5) (width 0.3) (layer F.Cu) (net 7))
 (segment (start 103.5 53.5) (end 102 52) (width 0.3) (layer F.Cu) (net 7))
 (segment (start 102.742081 44) (end 101.54 44) (width 0.3) (layer F.Cu) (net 7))
 (segment (start 103.54 42) (end 103.54 43.202081) (width 0.3) (layer F.Cu) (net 7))
 (segment (start 101 44.54) (end 101 47.5) (width 0.3) (layer F.Cu) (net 7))
 (segment (start 101 47.5) (end 101.376628 47.876628) (width 0.3) (layer F.Cu) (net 7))
 (segment (start 101.376628 48.376628) (end 102 49) (width 0.3) (layer F.Cu) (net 7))
 (segment (start 101.376628 47.876628) (end 101.376628 48.376628) (width 0.3) (layer F.Cu) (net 7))
 (segment (start 101.54 44) (end 101 44.54) (width 0.3) (layer F.Cu) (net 7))
 (segment (start 103.54 43.202081) (end 102.742081 44) (width 0.3) (layer F.Cu) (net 7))
 (segment (start 105.230001 42.849999) (end 106.08 42) (width 0.3) (layer B.Cu) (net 14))
 (segment (start 99.379999 48.700001) (end 105.230001 42.849999) (width 0.3) (layer B.Cu) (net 14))
 (segment (start 96.299999 48.700001) (end 99.379999 48.700001) (width 0.3) (layer B.Cu) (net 14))
 (segment (start 95 50) (end 96.299999 48.700001) (width 0.3) (layer B.Cu) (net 14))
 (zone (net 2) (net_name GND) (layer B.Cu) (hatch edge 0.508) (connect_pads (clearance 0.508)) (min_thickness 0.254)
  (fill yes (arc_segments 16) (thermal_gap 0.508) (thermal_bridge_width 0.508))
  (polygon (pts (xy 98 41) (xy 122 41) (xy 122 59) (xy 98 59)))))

